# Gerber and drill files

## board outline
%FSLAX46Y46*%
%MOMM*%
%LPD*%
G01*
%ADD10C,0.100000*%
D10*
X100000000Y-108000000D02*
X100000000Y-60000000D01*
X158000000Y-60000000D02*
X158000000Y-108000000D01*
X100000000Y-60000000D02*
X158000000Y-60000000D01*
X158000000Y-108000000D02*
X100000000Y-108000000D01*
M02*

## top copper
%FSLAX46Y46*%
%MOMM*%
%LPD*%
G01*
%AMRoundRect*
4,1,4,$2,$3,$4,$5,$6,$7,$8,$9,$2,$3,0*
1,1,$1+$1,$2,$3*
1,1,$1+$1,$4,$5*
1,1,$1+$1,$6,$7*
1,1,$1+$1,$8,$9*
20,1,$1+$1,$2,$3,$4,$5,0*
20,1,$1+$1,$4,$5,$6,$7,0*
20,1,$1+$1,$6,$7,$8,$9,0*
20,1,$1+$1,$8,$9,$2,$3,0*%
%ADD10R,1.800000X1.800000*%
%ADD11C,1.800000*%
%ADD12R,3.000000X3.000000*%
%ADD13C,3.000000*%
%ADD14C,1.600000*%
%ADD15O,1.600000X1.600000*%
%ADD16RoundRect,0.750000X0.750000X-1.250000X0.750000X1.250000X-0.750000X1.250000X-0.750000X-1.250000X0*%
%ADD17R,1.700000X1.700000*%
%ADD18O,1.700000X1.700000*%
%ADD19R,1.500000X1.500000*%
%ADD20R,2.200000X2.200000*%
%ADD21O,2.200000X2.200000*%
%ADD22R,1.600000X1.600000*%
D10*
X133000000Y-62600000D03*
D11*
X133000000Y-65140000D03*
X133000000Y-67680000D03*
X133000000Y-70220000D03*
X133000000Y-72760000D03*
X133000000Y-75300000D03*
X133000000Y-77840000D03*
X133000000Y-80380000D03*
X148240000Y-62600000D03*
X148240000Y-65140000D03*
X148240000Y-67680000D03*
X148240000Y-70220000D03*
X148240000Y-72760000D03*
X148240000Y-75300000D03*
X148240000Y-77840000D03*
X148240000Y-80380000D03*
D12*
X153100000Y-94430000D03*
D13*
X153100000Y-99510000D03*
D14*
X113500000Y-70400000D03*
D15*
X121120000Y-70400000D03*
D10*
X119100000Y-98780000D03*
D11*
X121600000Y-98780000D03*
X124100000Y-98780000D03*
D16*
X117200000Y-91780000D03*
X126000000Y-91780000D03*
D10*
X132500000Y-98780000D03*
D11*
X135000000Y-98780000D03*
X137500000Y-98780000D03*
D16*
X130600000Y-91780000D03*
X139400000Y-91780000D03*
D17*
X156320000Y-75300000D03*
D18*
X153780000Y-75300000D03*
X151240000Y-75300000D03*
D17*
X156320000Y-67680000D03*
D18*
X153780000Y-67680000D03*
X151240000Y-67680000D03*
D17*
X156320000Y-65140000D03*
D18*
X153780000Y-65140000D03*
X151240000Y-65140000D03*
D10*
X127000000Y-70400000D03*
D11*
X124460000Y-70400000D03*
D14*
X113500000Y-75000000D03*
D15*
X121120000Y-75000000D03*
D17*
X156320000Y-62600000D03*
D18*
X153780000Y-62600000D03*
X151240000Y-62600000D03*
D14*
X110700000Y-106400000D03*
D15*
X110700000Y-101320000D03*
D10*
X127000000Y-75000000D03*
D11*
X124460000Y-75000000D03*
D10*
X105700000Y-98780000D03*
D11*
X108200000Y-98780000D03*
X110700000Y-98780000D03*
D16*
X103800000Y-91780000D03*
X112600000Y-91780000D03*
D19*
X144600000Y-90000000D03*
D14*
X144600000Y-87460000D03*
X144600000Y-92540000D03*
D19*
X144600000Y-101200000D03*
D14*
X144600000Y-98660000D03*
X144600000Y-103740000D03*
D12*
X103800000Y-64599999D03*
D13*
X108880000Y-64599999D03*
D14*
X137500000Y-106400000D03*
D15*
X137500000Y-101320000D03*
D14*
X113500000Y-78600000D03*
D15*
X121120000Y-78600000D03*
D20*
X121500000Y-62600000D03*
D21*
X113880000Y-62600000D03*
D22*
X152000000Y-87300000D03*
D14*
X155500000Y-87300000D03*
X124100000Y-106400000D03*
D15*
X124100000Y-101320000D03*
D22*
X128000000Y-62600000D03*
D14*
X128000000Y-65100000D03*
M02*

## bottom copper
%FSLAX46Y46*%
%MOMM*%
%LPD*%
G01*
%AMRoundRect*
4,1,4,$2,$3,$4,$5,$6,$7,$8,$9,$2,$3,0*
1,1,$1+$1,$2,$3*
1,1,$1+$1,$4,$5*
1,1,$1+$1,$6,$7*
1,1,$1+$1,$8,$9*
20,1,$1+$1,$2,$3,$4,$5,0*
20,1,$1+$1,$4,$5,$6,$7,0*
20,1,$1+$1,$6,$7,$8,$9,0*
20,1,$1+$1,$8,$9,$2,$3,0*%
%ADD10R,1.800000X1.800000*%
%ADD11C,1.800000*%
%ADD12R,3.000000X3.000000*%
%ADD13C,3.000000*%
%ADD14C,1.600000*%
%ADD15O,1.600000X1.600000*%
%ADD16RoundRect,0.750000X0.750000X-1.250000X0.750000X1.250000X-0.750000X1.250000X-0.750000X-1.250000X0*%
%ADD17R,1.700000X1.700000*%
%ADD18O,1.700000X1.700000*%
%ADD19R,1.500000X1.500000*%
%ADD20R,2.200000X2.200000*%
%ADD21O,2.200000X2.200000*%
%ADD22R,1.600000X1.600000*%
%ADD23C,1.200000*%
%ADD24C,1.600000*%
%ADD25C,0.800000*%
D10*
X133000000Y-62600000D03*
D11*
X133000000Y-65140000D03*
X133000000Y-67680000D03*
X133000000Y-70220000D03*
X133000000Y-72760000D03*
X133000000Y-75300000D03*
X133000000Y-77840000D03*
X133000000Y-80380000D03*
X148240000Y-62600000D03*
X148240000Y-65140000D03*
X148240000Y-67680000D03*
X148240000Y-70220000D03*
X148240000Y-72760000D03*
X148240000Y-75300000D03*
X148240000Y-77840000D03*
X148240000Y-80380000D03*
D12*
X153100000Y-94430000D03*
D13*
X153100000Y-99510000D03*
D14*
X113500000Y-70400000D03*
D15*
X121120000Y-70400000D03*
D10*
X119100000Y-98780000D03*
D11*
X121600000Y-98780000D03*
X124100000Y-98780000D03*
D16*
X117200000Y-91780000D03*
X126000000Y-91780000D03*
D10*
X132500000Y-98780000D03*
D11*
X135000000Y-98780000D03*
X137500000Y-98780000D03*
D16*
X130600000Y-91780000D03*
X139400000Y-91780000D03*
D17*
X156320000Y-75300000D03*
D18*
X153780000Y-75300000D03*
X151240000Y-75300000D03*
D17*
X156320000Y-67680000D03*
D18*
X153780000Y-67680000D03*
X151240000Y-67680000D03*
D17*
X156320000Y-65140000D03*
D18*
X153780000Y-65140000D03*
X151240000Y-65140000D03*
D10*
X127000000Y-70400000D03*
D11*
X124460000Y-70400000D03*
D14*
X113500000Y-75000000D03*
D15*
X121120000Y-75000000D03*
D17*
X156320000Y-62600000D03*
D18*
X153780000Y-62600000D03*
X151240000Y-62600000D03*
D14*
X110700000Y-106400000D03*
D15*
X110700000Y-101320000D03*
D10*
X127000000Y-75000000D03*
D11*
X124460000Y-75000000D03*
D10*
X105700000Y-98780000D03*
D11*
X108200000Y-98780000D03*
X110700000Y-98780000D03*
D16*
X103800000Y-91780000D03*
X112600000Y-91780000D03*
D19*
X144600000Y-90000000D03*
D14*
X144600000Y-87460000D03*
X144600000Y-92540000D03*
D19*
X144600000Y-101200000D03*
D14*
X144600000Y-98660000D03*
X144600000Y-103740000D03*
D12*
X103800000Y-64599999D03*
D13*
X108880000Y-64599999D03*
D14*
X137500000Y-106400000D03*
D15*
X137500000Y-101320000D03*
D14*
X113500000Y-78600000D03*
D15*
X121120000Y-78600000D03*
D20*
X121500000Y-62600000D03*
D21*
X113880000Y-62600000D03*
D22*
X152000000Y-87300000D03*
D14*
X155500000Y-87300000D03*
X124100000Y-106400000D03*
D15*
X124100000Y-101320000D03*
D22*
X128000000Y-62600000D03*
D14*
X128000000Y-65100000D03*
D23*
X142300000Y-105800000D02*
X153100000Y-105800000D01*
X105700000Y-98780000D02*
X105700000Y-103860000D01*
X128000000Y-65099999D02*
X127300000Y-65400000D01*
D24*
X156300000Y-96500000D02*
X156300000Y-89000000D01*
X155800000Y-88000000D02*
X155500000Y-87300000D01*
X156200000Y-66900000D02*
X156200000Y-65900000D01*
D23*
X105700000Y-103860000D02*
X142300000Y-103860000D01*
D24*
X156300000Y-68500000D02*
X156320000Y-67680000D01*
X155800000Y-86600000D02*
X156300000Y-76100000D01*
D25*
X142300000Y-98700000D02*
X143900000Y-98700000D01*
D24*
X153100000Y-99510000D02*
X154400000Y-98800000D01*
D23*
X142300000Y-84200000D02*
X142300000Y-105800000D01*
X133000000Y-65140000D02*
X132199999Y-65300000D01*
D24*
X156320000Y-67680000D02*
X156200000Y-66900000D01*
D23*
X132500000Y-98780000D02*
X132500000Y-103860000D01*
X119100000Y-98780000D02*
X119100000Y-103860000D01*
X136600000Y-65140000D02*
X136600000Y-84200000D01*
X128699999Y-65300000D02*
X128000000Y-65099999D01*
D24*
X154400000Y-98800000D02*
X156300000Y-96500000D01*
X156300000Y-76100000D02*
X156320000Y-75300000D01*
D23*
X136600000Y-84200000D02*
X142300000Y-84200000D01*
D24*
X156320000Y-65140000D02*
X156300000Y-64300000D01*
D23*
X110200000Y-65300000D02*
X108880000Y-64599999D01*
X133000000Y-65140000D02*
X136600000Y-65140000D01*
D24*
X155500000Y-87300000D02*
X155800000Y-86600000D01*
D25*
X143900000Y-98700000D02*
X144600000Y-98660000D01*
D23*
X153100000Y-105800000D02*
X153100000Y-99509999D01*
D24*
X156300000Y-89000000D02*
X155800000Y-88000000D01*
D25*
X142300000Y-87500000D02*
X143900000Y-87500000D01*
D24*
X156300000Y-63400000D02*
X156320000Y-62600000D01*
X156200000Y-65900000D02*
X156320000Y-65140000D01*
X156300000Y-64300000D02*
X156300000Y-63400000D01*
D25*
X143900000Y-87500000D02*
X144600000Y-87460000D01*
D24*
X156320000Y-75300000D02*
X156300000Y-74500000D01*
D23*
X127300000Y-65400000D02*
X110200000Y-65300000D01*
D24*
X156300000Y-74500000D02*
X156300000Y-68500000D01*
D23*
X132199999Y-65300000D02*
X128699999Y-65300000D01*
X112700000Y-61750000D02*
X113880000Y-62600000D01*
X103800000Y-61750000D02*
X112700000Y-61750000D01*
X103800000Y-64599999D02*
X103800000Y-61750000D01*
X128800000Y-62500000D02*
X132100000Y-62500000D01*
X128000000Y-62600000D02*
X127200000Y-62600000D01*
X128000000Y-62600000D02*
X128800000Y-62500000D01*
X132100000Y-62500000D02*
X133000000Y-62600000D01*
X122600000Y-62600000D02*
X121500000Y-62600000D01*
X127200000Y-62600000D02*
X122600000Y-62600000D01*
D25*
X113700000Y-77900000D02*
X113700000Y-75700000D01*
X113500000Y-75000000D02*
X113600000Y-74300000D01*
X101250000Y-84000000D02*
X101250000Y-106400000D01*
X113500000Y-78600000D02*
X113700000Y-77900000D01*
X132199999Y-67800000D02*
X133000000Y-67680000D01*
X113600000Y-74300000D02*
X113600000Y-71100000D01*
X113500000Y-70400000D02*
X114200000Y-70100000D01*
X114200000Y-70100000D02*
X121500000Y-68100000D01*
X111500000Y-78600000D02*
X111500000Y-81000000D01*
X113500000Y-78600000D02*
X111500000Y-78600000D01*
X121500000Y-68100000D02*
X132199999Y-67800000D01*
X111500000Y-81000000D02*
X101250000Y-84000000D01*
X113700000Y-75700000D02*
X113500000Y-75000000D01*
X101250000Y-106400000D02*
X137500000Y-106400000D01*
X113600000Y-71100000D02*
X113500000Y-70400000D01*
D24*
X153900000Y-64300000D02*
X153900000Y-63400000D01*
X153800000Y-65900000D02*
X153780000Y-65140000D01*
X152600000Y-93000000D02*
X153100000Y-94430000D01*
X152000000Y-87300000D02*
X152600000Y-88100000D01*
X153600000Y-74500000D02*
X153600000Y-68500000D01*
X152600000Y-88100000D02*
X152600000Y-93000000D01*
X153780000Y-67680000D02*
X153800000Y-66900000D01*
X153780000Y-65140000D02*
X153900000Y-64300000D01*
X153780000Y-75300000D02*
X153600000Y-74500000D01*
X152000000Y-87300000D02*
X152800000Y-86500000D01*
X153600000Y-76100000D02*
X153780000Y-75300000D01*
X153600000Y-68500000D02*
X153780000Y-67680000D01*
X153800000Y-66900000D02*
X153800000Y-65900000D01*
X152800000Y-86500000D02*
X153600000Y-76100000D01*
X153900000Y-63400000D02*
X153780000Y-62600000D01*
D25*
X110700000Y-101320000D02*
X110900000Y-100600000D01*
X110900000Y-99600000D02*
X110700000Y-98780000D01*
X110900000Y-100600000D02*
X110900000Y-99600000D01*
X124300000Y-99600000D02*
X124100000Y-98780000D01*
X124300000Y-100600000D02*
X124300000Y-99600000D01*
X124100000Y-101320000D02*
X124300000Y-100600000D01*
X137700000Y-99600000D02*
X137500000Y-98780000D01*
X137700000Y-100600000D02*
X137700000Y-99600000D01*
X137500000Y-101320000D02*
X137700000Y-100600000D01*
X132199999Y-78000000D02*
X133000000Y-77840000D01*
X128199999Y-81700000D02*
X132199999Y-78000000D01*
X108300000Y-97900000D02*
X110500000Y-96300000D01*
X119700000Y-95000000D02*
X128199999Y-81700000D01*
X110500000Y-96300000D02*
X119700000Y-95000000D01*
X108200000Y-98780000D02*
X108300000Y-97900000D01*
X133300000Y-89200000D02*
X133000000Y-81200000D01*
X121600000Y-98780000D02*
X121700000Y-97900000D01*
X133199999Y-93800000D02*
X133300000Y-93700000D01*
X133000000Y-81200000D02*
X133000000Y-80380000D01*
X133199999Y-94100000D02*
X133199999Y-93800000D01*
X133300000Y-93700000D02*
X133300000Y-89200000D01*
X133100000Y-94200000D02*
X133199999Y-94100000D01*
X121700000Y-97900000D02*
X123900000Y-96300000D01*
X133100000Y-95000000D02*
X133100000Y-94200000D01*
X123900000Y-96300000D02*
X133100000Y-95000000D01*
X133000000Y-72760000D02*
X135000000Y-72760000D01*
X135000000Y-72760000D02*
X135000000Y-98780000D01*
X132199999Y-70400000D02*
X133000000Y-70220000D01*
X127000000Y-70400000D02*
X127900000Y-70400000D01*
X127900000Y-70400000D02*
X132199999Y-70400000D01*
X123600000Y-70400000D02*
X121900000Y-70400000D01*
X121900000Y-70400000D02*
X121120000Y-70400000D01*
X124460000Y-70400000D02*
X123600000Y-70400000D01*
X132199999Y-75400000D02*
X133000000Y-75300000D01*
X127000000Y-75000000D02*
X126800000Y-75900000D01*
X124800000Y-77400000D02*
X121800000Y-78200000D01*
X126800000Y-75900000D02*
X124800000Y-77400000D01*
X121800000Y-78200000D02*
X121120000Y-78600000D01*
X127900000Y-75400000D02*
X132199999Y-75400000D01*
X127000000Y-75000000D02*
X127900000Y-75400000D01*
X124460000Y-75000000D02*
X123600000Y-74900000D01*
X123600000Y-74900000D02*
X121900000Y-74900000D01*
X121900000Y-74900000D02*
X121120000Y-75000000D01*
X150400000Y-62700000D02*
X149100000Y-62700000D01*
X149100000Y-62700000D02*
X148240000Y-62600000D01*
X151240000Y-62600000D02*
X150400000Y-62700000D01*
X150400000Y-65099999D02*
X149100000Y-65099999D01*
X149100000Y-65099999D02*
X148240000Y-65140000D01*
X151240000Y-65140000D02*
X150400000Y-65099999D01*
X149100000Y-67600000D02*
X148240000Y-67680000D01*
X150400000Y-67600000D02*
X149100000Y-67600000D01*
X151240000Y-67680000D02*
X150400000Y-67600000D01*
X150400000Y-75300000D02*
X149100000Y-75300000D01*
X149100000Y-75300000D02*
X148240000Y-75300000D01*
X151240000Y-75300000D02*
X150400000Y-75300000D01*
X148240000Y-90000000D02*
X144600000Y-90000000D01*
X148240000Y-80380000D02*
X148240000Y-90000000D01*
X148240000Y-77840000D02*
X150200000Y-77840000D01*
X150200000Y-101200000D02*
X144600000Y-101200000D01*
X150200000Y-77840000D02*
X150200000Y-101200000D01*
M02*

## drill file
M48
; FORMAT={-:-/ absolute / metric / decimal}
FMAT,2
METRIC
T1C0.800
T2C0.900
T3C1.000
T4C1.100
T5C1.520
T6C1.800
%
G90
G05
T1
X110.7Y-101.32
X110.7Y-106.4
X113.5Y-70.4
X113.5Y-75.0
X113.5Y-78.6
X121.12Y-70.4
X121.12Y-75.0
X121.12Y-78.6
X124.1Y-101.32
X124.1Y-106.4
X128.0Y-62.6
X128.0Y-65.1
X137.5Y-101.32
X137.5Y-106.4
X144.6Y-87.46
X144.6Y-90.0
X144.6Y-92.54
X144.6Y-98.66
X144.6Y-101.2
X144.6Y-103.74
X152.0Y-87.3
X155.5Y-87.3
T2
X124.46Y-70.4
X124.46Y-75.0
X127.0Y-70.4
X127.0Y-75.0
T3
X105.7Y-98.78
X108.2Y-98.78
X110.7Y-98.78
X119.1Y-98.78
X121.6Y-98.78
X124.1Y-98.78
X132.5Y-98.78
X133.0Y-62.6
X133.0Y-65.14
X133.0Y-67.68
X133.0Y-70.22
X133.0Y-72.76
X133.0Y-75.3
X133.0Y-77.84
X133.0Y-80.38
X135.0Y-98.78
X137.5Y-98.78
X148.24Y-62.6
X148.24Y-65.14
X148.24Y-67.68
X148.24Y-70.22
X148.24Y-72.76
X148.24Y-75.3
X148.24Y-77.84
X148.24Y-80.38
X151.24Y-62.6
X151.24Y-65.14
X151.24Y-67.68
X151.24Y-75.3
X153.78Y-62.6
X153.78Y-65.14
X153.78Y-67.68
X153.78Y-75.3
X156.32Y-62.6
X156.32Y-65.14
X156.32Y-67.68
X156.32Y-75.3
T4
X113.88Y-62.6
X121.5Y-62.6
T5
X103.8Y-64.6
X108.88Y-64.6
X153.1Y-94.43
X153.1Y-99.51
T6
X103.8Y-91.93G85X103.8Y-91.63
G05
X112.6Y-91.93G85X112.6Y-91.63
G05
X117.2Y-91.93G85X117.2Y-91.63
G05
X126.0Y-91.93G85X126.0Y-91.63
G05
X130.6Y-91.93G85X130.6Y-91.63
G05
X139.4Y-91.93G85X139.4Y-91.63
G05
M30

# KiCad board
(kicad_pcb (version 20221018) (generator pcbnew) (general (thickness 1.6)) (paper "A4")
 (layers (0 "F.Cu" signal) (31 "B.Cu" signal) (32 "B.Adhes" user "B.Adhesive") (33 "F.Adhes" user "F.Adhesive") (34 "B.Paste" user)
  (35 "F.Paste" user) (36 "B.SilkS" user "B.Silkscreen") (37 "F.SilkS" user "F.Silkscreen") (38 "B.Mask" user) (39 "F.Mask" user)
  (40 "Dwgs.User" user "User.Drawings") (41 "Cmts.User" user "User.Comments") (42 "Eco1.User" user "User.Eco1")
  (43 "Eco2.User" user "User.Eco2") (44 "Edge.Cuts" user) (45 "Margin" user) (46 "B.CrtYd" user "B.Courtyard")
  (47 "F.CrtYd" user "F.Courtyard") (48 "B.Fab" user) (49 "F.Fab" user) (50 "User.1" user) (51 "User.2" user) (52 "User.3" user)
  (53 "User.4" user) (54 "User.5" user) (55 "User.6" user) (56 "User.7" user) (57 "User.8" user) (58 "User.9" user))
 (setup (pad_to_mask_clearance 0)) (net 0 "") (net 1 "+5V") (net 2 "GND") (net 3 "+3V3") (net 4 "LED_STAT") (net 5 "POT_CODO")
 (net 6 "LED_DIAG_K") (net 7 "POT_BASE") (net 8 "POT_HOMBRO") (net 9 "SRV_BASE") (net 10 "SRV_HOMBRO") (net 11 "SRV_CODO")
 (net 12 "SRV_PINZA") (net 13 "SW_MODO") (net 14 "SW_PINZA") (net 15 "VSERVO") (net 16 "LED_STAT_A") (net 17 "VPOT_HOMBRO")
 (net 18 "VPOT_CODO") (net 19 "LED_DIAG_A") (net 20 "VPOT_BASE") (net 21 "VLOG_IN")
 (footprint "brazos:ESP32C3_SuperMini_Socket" (layer "F.Cu") (at 133 62.6)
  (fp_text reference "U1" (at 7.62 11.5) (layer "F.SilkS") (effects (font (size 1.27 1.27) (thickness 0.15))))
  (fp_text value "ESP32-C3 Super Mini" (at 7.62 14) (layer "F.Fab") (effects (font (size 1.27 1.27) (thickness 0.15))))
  (pad "1" thru_hole rect (at 0 0) (size 1.8 1.8) (drill 1) (layers "*.Cu" "*.Mask") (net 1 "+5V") (thermal_bridge_angle 45))
  (pad "2" thru_hole circle (at 0 2.54) (size 1.8 1.8) (drill 1) (layers "*.Cu" "*.Mask") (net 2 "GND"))
  (pad "3" thru_hole circle (at 0 5.08) (size 1.8 1.8) (drill 1) (layers "*.Cu" "*.Mask") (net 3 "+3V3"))
  (pad "4" thru_hole circle (at 0 7.62) (size 1.8 1.8) (drill 1) (layers "*.Cu" "*.Mask") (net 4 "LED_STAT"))
  (pad "5" thru_hole circle (at 0 10.16) (size 1.8 1.8) (drill 1) (layers "*.Cu" "*.Mask") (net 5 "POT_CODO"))
  (pad "6" thru_hole circle (at 0 12.7) (size 1.8 1.8) (drill 1) (layers "*.Cu" "*.Mask") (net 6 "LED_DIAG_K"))
  (pad "7" thru_hole circle (at 0 15.24) (size 1.8 1.8) (drill 1) (layers "*.Cu" "*.Mask") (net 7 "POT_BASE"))
  (pad "8" thru_hole circle (at 0 17.78) (size 1.8 1.8) (drill 1) (layers "*.Cu" "*.Mask") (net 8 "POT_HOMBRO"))
  (pad "9" thru_hole circle (at 15.24 0) (size 1.8 1.8) (drill 1) (layers "*.Cu" "*.Mask") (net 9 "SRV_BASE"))
  (pad "10" thru_hole circle (at 15.24 2.54) (size 1.8 1.8) (drill 1) (layers "*.Cu" "*.Mask") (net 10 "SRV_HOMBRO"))
  (pad "11" thru_hole circle (at 15.24 5.08) (size 1.8 1.8) (drill 1) (layers "*.Cu" "*.Mask") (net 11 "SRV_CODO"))
  (pad "12" thru_hole circle (at 15.24 7.62) (size 1.8 1.8) (drill 1) (layers "*.Cu" "*.Mask"))
  (pad "13" thru_hole circle (at 15.24 10.16) (size 1.8 1.8) (drill 1) (layers "*.Cu" "*.Mask"))
  (pad "14" thru_hole circle (at 15.24 12.7) (size 1.8 1.8) (drill 1) (layers "*.Cu" "*.Mask") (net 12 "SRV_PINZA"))
  (pad "15" thru_hole circle (at 15.24 15.24) (size 1.8 1.8) (drill 1) (layers "*.Cu" "*.Mask") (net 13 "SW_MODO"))
  (pad "16" thru_hole circle (at 15.24 17.78) (size 1.8 1.8) (drill 1) (layers "*.Cu" "*.Mask") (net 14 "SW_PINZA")))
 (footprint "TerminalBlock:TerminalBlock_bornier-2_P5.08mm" (layer "F.Cu") (at 153.1 94.43 -90)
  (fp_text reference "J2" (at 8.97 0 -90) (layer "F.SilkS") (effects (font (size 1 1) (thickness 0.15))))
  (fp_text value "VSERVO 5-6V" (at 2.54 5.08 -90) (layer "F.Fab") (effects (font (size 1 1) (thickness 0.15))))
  (pad "1" thru_hole rect (at 0 0 270) (size 3 3) (drill 1.52) (layers "*.Cu" "*.Mask") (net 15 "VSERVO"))
  (pad "2" thru_hole circle (at 5.08 0 270) (size 3 3) (drill 1.52) (layers "*.Cu" "*.Mask") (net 2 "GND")))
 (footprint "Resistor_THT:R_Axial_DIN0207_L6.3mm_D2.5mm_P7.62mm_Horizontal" (layer "F.Cu") (at 113.5 70.4)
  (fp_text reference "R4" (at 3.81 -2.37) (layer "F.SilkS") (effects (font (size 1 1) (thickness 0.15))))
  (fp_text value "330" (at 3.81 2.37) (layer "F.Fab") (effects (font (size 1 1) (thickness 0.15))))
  (pad "1" thru_hole circle (at 0 0) (size 1.6 1.6) (drill 0.8) (layers "*.Cu" "*.Mask") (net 3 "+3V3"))
  (pad "2" thru_hole oval (at 7.62 0) (size 1.6 1.6) (drill 0.8) (layers "*.Cu" "*.Mask") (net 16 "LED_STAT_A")))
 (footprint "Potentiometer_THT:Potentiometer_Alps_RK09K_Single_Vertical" (layer "F.Cu") (at 119.1 98.78 90)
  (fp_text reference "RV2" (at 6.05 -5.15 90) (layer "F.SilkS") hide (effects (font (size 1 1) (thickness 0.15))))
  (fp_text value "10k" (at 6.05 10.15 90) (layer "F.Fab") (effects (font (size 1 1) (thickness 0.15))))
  (pad "1" thru_hole rect (at 0 0 90) (size 1.8 1.8) (drill 1) (layers "*.Cu" "*.Mask") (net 2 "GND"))
  (pad "2" thru_hole circle (at 0 2.5 90) (size 1.8 1.8) (drill 1) (layers "*.Cu" "*.Mask") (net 8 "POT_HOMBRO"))
  (pad "3" thru_hole circle (at 0 5 90) (size 1.8 1.8) (drill 1) (layers "*.Cu" "*.Mask") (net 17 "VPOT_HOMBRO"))
  (pad "MP" thru_hole roundrect (at 7 -1.9 90) (size 4 3) (drill oval 2.1 1.8) (layers "*.Cu" "*.Mask") (roundrect_rratio 0.25))
  (pad "MP" thru_hole roundrect (at 7 6.9 90) (size 4 3) (drill oval 2.1 1.8) (layers "*.Cu" "*.Mask") (roundrect_rratio 0.25)))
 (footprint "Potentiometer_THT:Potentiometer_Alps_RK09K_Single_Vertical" (layer "F.Cu") (at 132.5 98.78 90)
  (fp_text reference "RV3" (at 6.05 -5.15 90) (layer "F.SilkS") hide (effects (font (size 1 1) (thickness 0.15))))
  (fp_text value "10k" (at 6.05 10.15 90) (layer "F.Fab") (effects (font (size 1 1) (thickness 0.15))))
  (pad "1" thru_hole rect (at 0 0 90) (size 1.8 1.8) (drill 1) (layers "*.Cu" "*.Mask") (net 2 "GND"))
  (pad "2" thru_hole circle (at 0 2.5 90) (size 1.8 1.8) (drill 1) (layers "*.Cu" "*.Mask") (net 5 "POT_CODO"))
  (pad "3" thru_hole circle (at 0 5 90) (size 1.8 1.8) (drill 1) (layers "*.Cu" "*.Mask") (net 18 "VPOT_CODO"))
  (pad "MP" thru_hole roundrect (at 7 -1.9 90) (size 4 3) (drill oval 2.1 1.8) (layers "*.Cu" "*.Mask") (roundrect_rratio 0.25))
  (pad "MP" thru_hole roundrect (at 7 6.9 90) (size 4 3) (drill oval 2.1 1.8) (layers "*.Cu" "*.Mask") (roundrect_rratio 0.25)))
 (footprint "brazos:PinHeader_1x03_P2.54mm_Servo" (layer "F.Cu") (at 156.32 75.3 -90)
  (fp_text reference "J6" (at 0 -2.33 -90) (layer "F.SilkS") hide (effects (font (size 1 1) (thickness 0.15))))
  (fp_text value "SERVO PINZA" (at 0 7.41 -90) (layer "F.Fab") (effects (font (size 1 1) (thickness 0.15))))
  (pad "1" thru_hole rect (at 0 0 270) (size 1.7 1.7) (drill 1) (layers "*.Cu" "*.Mask") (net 2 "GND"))
  (pad "2" thru_hole oval (at 0 2.54 270) (size 1.7 1.7) (drill 1) (layers "*.Cu" "*.Mask") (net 15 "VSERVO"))
  (pad "3" thru_hole oval (at 0 5.08 270) (size 1.7 1.7) (drill 1) (layers "*.Cu" "*.Mask") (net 12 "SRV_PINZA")))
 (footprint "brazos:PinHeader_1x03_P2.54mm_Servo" (layer "F.Cu") (at 156.32 67.68 -90)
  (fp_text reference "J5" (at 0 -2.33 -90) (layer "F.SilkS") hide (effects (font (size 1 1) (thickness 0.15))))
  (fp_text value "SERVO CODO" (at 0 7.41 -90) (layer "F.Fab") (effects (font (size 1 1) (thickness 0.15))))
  (pad "1" thru_hole rect (at 0 0 270) (size 1.7 1.7) (drill 1) (layers "*.Cu" "*.Mask") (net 2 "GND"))
  (pad "2" thru_hole oval (at 0 2.54 270) (size 1.7 1.7) (drill 1) (layers "*.Cu" "*.Mask") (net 15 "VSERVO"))
  (pad "3" thru_hole oval (at 0 5.08 270) (size 1.7 1.7) (drill 1) (layers "*.Cu" "*.Mask") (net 11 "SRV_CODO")))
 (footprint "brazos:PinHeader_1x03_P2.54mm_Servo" (layer "F.Cu") (at 156.32 65.14 -90)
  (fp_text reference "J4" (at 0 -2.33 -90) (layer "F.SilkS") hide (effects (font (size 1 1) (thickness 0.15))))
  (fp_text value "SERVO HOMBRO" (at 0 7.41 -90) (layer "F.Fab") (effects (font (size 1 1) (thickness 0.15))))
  (pad "1" thru_hole rect (at 0 0 270) (size 1.7 1.7) (drill 1) (layers "*.Cu" "*.Mask") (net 2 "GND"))
  (pad "2" thru_hole oval (at 0 2.54 270) (size 1.7 1.7) (drill 1) (layers "*.Cu" "*.Mask") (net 15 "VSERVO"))
  (pad "3" thru_hole oval (at 0 5.08 270) (size 1.7 1.7) (drill 1) (layers "*.Cu" "*.Mask") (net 10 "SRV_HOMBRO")))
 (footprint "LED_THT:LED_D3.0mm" (layer "F.Cu") (at 127 70.4 180)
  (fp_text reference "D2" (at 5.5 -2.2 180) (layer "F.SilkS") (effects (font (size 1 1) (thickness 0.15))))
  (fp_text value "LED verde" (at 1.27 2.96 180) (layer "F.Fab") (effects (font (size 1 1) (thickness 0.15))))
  (pad "1" thru_hole rect (at 0 0 180) (size 1.8 1.8) (drill 0.9) (layers "*.Cu" "*.Mask") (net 4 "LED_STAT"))
  (pad "2" thru_hole circle (at 2.54 0 180) (size 1.8 1.8) (drill 0.9) (layers "*.Cu" "*.Mask") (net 16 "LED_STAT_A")))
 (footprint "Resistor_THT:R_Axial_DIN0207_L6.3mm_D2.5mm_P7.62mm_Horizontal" (layer "F.Cu") (at 113.5 75)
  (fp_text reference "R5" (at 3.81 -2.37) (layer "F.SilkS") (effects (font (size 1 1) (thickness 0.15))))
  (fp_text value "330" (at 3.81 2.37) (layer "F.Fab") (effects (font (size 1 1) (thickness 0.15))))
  (pad "1" thru_hole circle (at 0 0) (size 1.6 1.6) (drill 0.8) (layers "*.Cu" "*.Mask") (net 3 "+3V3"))
  (pad "2" thru_hole oval (at 7.62 0) (size 1.6 1.6) (drill 0.8) (layers "*.Cu" "*.Mask") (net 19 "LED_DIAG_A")))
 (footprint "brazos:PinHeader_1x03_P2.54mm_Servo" (layer "F.Cu") (at 156.32 62.6 -90)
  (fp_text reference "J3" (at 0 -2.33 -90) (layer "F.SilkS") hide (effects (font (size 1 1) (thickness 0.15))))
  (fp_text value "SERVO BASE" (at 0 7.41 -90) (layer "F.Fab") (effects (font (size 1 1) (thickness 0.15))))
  (pad "1" thru_hole rect (at 0 0 270) (size 1.7 1.7) (drill 1) (layers "*.Cu" "*.Mask") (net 2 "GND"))
  (pad "2" thru_hole oval (at 0 2.54 270) (size 1.7 1.7) (drill 1) (layers "*.Cu" "*.Mask") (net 15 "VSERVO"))
  (pad "3" thru_hole oval (at 0 5.08 270) (size 1.7 1.7) (drill 1) (layers "*.Cu" "*.Mask") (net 9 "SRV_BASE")))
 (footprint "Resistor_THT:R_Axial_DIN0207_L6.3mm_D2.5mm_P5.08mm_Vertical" (layer "F.Cu") (at 110.7 106.4 90)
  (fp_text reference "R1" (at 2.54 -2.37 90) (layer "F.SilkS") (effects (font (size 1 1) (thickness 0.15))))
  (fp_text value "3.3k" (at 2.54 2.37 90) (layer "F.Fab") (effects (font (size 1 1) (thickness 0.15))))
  (pad "1" thru_hole circle (at 0 0 90) (size 1.6 1.6) (drill 0.8) (layers "*.Cu" "*.Mask") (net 3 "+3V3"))
  (pad "2" thru_hole oval (at 5.08 0 90) (size 1.6 1.6) (drill 0.8) (layers "*.Cu" "*.Mask") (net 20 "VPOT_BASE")))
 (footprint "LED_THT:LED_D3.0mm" (layer "F.Cu") (at 127 75 180)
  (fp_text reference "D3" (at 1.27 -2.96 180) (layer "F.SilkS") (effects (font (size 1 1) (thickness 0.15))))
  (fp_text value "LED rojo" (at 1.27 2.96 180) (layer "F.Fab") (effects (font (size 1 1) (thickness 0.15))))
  (pad "1" thru_hole rect (at 0 0 180) (size 1.8 1.8) (drill 0.9) (layers "*.Cu" "*.Mask") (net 6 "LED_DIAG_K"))
  (pad "2" thru_hole circle (at 2.54 0 180) (size 1.8 1.8) (drill 0.9) (layers "*.Cu" "*.Mask") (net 19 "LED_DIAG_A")))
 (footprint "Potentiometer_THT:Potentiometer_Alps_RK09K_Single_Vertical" (layer "F.Cu") (at 105.7 98.78 90)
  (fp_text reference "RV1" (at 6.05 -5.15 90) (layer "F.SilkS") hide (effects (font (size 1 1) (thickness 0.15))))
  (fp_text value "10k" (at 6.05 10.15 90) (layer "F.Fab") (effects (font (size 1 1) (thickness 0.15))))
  (pad "1" thru_hole rect (at 0 0 90) (size 1.8 1.8) (drill 1) (layers "*.Cu" "*.Mask") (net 2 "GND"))
  (pad "2" thru_hole circle (at 0 2.5 90) (size 1.8 1.8) (drill 1) (layers "*.Cu" "*.Mask") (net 7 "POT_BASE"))
  (pad "3" thru_hole circle (at 0 5 90) (size 1.8 1.8) (drill 1) (layers "*.Cu" "*.Mask") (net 20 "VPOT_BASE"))
  (pad "MP" thru_hole roundrect (at 7 -1.9 90) (size 4 3) (drill oval 2.1 1.8) (layers "*.Cu" "*.Mask") (roundrect_rratio 0.25))
  (pad "MP" thru_hole roundrect (at 7 6.9 90) (size 4 3) (drill oval 2.1 1.8) (layers "*.Cu" "*.Mask") (roundrect_rratio 0.25)))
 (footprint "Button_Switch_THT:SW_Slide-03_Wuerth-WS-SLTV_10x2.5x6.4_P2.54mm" (layer "F.Cu") (at 144.6 90 -90)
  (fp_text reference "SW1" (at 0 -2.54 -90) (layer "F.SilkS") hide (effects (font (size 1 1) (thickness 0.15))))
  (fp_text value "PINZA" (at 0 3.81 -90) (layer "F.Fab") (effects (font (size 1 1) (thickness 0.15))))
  (pad "1" thru_hole rect (at 0 0 270) (size 1.5 1.5) (drill 0.8) (layers "*.Cu" "*.Mask") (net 14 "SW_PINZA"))
  (pad "2" thru_hole circle (at -2.54 0 270) (size 1.6 1.6) (drill 0.8) (layers "*.Cu" "*.Mask") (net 2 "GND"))
  (pad "3" thru_hole circle (at 2.54 0 270) (size 1.6 1.6) (drill 0.8) (layers "*.Cu" "*.Mask")))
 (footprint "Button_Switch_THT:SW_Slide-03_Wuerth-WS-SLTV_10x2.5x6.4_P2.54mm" (layer "F.Cu") (at 144.6 101.2 -90)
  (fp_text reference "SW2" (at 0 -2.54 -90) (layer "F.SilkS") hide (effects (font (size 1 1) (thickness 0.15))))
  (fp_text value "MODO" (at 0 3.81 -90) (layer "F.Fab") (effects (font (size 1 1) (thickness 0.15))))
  (pad "1" thru_hole rect (at 0 0 270) (size 1.5 1.5) (drill 0.8) (layers "*.Cu" "*.Mask") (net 13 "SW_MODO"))
  (pad "2" thru_hole circle (at -2.54 0 270) (size 1.6 1.6) (drill 0.8) (layers "*.Cu" "*.Mask") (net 2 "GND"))
  (pad "3" thru_hole circle (at 2.54 0 270) (size 1.6 1.6) (drill 0.8) (layers "*.Cu" "*.Mask")))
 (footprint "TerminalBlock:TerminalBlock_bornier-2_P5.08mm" (layer "F.Cu") (at 103.8 64.599999)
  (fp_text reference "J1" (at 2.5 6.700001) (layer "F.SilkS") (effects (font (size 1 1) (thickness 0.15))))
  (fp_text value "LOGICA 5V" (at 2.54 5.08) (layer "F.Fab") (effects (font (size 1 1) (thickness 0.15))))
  (pad "1" thru_hole rect (at 0 0) (size 3 3) (drill 1.52) (layers "*.Cu" "*.Mask") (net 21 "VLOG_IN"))
  (pad "2" thru_hole circle (at 5.08 0) (size 3 3) (drill 1.52) (layers "*.Cu" "*.Mask") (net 2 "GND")))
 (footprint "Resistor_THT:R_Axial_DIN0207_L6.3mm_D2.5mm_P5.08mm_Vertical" (layer "F.Cu") (at 137.5 106.4 90)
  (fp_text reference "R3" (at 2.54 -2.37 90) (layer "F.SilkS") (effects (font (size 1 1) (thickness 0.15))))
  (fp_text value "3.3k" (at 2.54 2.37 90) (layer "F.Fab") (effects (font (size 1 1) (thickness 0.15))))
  (pad "1" thru_hole circle (at 0 0 90) (size 1.6 1.6) (drill 0.8) (layers "*.Cu" "*.Mask") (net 3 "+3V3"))
  (pad "2" thru_hole oval (at 5.08 0 90) (size 1.6 1.6) (drill 0.8) (layers "*.Cu" "*.Mask") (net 18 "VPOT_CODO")))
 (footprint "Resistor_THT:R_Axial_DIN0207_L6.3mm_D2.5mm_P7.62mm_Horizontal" (layer "F.Cu") (at 113.5 78.6)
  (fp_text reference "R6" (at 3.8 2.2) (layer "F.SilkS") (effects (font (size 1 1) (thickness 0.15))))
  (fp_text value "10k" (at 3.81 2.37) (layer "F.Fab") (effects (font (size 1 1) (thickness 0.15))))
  (pad "1" thru_hole circle (at 0 0) (size 1.6 1.6) (drill 0.8) (layers "*.Cu" "*.Mask") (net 3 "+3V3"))
  (pad "2" thru_hole oval (at 7.62 0) (size 1.6 1.6) (drill 0.8) (layers "*.Cu" "*.Mask") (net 6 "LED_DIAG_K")))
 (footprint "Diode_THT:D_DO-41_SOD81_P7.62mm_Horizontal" (layer "F.Cu") (at 121.5 62.6 180)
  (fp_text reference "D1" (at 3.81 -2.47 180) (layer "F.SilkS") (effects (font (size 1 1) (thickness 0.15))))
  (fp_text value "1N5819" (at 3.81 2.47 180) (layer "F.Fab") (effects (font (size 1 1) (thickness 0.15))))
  (pad "1" thru_hole rect (at 0 0 180) (size 2.2 2.2) (drill 1.1) (layers "*.Cu" "*.Mask") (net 1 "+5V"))
  (pad "2" thru_hole oval (at 7.62 0 180) (size 2.2 2.2) (drill 1.1) (layers "*.Cu" "*.Mask") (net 21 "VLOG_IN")))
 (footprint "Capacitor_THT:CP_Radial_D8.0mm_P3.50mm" (layer "F.Cu") (at 152 87.3)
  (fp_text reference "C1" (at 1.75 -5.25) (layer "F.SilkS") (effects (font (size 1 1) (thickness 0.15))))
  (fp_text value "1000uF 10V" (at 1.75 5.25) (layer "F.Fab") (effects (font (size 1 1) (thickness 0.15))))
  (pad "1" thru_hole rect (at 0 0) (size 1.6 1.6) (drill 0.8) (layers "*.Cu" "*.Mask") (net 15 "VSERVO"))
  (pad "2" thru_hole circle (at 3.5 0) (size 1.6 1.6) (drill 0.8) (layers "*.Cu" "*.Mask") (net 2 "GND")))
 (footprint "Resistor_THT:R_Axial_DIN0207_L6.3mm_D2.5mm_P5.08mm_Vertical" (layer "F.Cu") (at 124.1 106.4 90)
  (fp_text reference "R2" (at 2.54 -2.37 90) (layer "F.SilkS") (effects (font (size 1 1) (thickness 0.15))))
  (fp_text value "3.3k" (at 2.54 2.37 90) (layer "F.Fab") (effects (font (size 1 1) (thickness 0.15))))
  (pad "1" thru_hole circle (at 0 0 90) (size 1.6 1.6) (drill 0.8) (layers "*.Cu" "*.Mask") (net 3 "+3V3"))
  (pad "2" thru_hole oval (at 5.08 0 90) (size 1.6 1.6) (drill 0.8) (layers "*.Cu" "*.Mask") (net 17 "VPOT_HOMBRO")))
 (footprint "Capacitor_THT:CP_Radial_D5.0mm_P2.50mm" (layer "F.Cu") (at 128 62.6 -90)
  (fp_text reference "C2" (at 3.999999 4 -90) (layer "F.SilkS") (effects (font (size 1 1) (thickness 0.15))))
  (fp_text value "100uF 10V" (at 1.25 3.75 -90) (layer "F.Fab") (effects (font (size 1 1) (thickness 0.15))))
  (pad "1" thru_hole rect (at 0 0 270) (size 1.6 1.6) (drill 0.8) (layers "*.Cu" "*.Mask") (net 1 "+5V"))
  (pad "2" thru_hole circle (at 2.5 0 270) (size 1.6 1.6) (drill 0.8) (layers "*.Cu" "*.Mask") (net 2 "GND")))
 (gr_line (start 100 108) (end 100 60) (stroke (width 0.1) (type default)) (layer "Edge.Cuts"))
 (gr_line (start 158 60) (end 158 108) (stroke (width 0.1) (type default)) (layer "Edge.Cuts"))
 (gr_line (start 100 60) (end 158 60) (stroke (width 0.1) (type default)) (layer "Edge.Cuts"))
 (gr_line (start 158 108) (end 100 108) (stroke (width 0.1) (type default)) (layer "Edge.Cuts"))
 (segment (start 142.3 105.8) (end 153.1 105.8) (width 1.2) (layer "B.Cu") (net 2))
 (segment (start 105.7 98.78) (end 105.7 103.86) (width 1.2) (layer "B.Cu") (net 2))
 (segment (start 128 65.099999) (end 127.3 65.4) (width 1.2) (layer "B.Cu") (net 2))
 (segment (start 156.3 96.5) (end 156.3 89) (width 1.6) (layer "B.Cu") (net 2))
 (segment (start 155.8 88) (end 155.5 87.3) (width 1.6) (layer "B.Cu") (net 2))
 (segment (start 156.2 66.9) (end 156.2 65.9) (width 1.6) (layer "B.Cu") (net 2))
 (segment (start 105.7 103.86) (end 142.3 103.86) (width 1.2) (layer "B.Cu") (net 2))
 (segment (start 156.3 68.5) (end 156.32 67.68) (width 1.6) (layer "B.Cu") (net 2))
 (segment (start 155.8 86.6) (end 156.3 76.1) (width 1.6) (layer "B.Cu") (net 2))
 (segment (start 142.3 98.7) (end 143.9 98.7) (width 0.8) (layer "B.Cu") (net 2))
 (segment (start 153.1 99.51) (end 154.4 98.8) (width 1.6) (layer "B.Cu") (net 2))
 (segment (start 142.3 84.2) (end 142.3 105.8) (width 1.2) (layer "B.Cu") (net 2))
 (segment (start 133 65.14) (end 132.199999 65.3) (width 1.2) (layer "B.Cu") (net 2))
 (segment (start 156.32 67.68) (end 156.2 66.9) (width 1.6) (layer "B.Cu") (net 2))
 (segment (start 132.5 98.78) (end 132.5 103.86) (width 1.2) (layer "B.Cu") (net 2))
 (segment (start 119.1 98.78) (end 119.1 103.86) (width 1.2) (layer "B.Cu") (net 2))
 (segment (start 136.6 65.14) (end 136.6 84.2) (width 1.2) (layer "B.Cu") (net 2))
 (segment (start 128.699999 65.3) (end 128 65.099999) (width 1.2) (layer "B.Cu") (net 2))
 (segment (start 154.4 98.8) (end 156.3 96.5) (width 1.6) (layer "B.Cu") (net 2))
 (segment (start 156.3 76.1) (end 156.32 75.3) (width 1.6) (layer "B.Cu") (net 2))
 (segment (start 136.6 84.2) (end 142.3 84.2) (width 1.2) (layer "B.Cu") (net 2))
 (segment (start 156.32 65.14) (end 156.3 64.3) (width 1.6) (layer "B.Cu") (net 2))
 (segment (start 110.2 65.3) (end 108.88 64.599999) (width 1.2) (layer "B.Cu") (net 2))
 (segment (start 133 65.14) (end 136.6 65.14) (width 1.2) (layer "B.Cu") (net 2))
 (segment (start 155.5 87.3) (end 155.8 86.6) (width 1.6) (layer "B.Cu") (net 2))
 (segment (start 143.9 98.7) (end 144.6 98.66) (width 0.8) (layer "B.Cu") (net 2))
 (segment (start 153.1 105.8) (end 153.1 99.509999) (width 1.2) (layer "B.Cu") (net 2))
 (segment (start 156.3 89) (end 155.8 88) (width 1.6) (layer "B.Cu") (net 2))
 (segment (start 142.3 87.5) (end 143.9 87.5) (width 0.8) (layer "B.Cu") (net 2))
 (segment (start 156.3 63.4) (end 156.32 62.6) (width 1.6) (layer "B.Cu") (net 2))
 (segment (start 156.2 65.9) (end 156.32 65.14) (width 1.6) (layer "B.Cu") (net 2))
 (segment (start 156.3 64.3) (end 156.3 63.4) (width 1.6) (layer "B.Cu") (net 2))
 (segment (start 143.9 87.5) (end 144.6 87.46) (width 0.8) (layer "B.Cu") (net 2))
 (segment (start 156.32 75.3) (end 156.3 74.5) (width 1.6) (layer "B.Cu") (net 2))
 (segment (start 127.3 65.4) (end 110.2 65.3) (width 1.2) (layer "B.Cu") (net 2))
 (segment (start 156.3 74.5) (end 156.3 68.5) (width 1.6) (layer "B.Cu") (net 2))
 (segment (start 132.199999 65.3) (end 128.699999 65.3) (width 1.2) (layer "B.Cu") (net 2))
 (segment (start 112.7 61.75) (end 113.88 62.6) (width 1.2) (layer "B.Cu") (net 21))
 (segment (start 103.8 61.75) (end 112.7 61.75) (width 1.2) (layer "B.Cu") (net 21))
 (segment (start 103.8 64.599999) (end 103.8 61.75) (width 1.2) (layer "B.Cu") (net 21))
 (segment (start 128.8 62.5) (end 132.1 62.5) (width 1.2) (layer "B.Cu") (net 1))
 (segment (start 128 62.6) (end 127.2 62.6) (width 1.2) (layer "B.Cu") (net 1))
 (segment (start 128 62.6) (end 128.8 62.5) (width 1.2) (layer "B.Cu") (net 1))
 (segment (start 132.1 62.5) (end 133 62.6) (width 1.2) (layer "B.Cu") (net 1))
 (segment (start 122.6 62.6) (end 121.5 62.6) (width 1.2) (layer "B.Cu") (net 1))
 (segment (start 127.2 62.6) (end 122.6 62.6) (width 1.2) (layer "B.Cu") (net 1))
 (segment (start 113.7 77.9) (end 113.7 75.7) (width 0.8) (layer "B.Cu") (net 3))
 (segment (start 113.5 75) (end 113.6 74.3) (width 0.8) (layer "B.Cu") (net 3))
 (segment (start 101.25 84) (end 101.25 106.4) (width 0.8) (layer "B.Cu") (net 3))
 (segment (start 113.5 78.6) (end 113.7 77.9) (width 0.8) (layer "B.Cu") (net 3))
 (segment (start 132.199999 67.8) (end 133 67.68) (width 0.8) (layer "B.Cu") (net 3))
 (segment (start 113.6 74.3) (end 113.6 71.1) (width 0.8) (layer "B.Cu") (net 3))
 (segment (start 113.5 70.4) (end 114.2 70.1) (width 0.8) (layer "B.Cu") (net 3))
 (segment (start 114.2 70.1) (end 121.5 68.1) (width 0.8) (layer "B.Cu") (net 3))
 (segment (start 111.5 78.6) (end 111.5 81) (width 0.8) (layer "B.Cu") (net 3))
 (segment (start 113.5 78.6) (end 111.5 78.6) (width 0.8) (layer "B.Cu") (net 3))
 (segment (start 121.5 68.1) (end 132.199999 67.8) (width 0.8) (layer "B.Cu") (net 3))
 (segment (start 111.5 81) (end 101.25 84) (width 0.8) (layer "B.Cu") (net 3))
 (segment (start 113.7 75.7) (end 113.5 75) (width 0.8) (layer "B.Cu") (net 3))
 (segment (start 101.25 106.4) (end 137.5 106.4) (width 0.8) (layer "B.Cu") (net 3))
 (segment (start 113.6 71.1) (end 113.5 70.4) (width 0.8) (layer "B.Cu") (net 3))
 (segment (start 153.9 64.3) (end 153.9 63.4) (width 1.6) (layer "B.Cu") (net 15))
 (segment (start 153.8 65.9) (end 153.78 65.14) (width 1.6) (layer "B.Cu") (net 15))
 (segment (start 152.6 93) (end 153.1 94.43) (width 1.6) (layer "B.Cu") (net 15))
 (segment (start 152 87.3) (end 152.6 88.1) (width 1.6) (layer "B.Cu") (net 15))
 (segment (start 153.6 74.5) (end 153.6 68.5) (width 1.6) (layer "B.Cu") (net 15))
 (segment (start 152.6 88.1) (end 152.6 93) (width 1.6) (layer "B.Cu") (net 15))
 (segment (start 153.78 67.68) (end 153.8 66.9) (width 1.6) (layer "B.Cu") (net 15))
 (segment (start 153.78 65.14) (end 153.9 64.3) (width 1.6) (layer "B.Cu") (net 15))
 (segment (start 153.78 75.3) (end 153.6 74.5) (width 1.6) (layer "B.Cu") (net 15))
 (segment (start 152 87.3) (end 152.8 86.5) (width 1.6) (layer "B.Cu") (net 15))
 (segment (start 153.6 76.1) (end 153.78 75.3) (width 1.6) (layer "B.Cu") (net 15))
 (segment (start 153.6 68.5) (end 153.78 67.68) (width 1.6) (layer "B.Cu") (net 15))
 (segment (start 153.8 66.9) (end 153.8 65.9) (width 1.6) (layer "B.Cu") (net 15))
 (segment (start 152.8 86.5) (end 153.6 76.1) (width 1.6) (layer "B.Cu") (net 15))
 (segment (start 153.9 63.4) (end 153.78 62.6) (width 1.6) (layer "B.Cu") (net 15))
 (segment (start 110.7 101.32) (end 110.9 100.6) (width 0.8) (layer "B.Cu") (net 20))
 (segment (start 110.9 99.6) (end 110.7 98.78) (width 0.8) (layer "B.Cu") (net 20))
 (segment (start 110.9 100.6) (end 110.9 99.6) (width 0.8) (layer "B.Cu") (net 20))
 (segment (start 124.3 99.6) (end 124.1 98.78) (width 0.8) (layer "B.Cu") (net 17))
 (segment (start 124.3 100.6) (end 124.3 99.6) (width 0.8) (layer "B.Cu") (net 17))
 (segment (start 124.1 101.32) (end 124.3 100.6) (width 0.8) (layer "B.Cu") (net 17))
 (segment (start 137.7 99.6) (end 137.5 98.78) (width 0.8) (layer "B.Cu") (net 18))
 (segment (start 137.7 100.6) (end 137.7 99.6) (width 0.8) (layer "B.Cu") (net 18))
 (segment (start 137.5 101.32) (end 137.7 100.6) (width 0.8) (layer "B.Cu") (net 18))
 (segment (start 132.199999 78) (end 133 77.84) (width 0.8) (layer "B.Cu") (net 7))
 (segment (start 128.199999 81.7) (end 132.199999 78) (width 0.8) (layer "B.Cu") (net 7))
 (segment (start 108.3 97.9) (end 110.5 96.3) (width 0.8) (layer "B.Cu") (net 7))
 (segment (start 119.7 95) (end 128.199999 81.7) (width 0.8) (layer "B.Cu") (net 7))
 (segment (start 110.5 96.3) (end 119.7 95) (width 0.8) (layer "B.Cu") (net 7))
 (segment (start 108.2 98.78) (end 108.3 97.9) (width 0.8) (layer "B.Cu") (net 7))
 (segment (start 133.3 89.2) (end 133 81.2) (width 0.8) (layer "B.Cu") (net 8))
 (segment (start 121.6 98.78) (end 121.7 97.9) (width 0.8) (layer "B.Cu") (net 8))
 (segment (start 133.199999 93.8) (end 133.3 93.7) (width 0.8) (layer "B.Cu") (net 8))
 (segment (start 133 81.2) (end 133 80.38) (width 0.8) (layer "B.Cu") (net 8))
 (segment (start 133.199999 94.1) (end 133.199999 93.8) (width 0.8) (layer "B.Cu") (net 8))
 (segment (start 133.3 93.7) (end 133.3 89.2) (width 0.8) (layer "B.Cu") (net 8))
 (segment (start 133.1 94.2) (end 133.199999 94.1) (width 0.8) (layer "B.Cu") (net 8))
 (segment (start 121.7 97.9) (end 123.9 96.3) (width 0.8) (layer "B.Cu") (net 8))
 (segment (start 133.1 95) (end 133.1 94.2) (width 0.8) (layer "B.Cu") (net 8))
 (segment (start 123.9 96.3) (end 133.1 95) (width 0.8) (layer "B.Cu") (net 8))
 (segment (start 133 72.76) (end 135 72.76) (width 0.8) (layer "B.Cu") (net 5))
 (segment (start 135 72.76) (end 135 98.78) (width 0.8) (layer "B.Cu") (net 5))
 (segment (start 132.199999 70.4) (end 133 70.22) (width 0.8) (layer "B.Cu") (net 4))
 (segment (start 127 70.4) (end 127.9 70.4) (width 0.8) (layer "B.Cu") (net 4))
 (segment (start 127.9 70.4) (end 132.199999 70.4) (width 0.8) (layer "B.Cu") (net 4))
 (segment (start 123.6 70.4) (end 121.9 70.4) (width 0.8) (layer "B.Cu") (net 16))
 (segment (start 121.9 70.4) (end 121.12 70.4) (width 0.8) (layer "B.Cu") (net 16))
 (segment (start 124.46 70.4) (end 123.6 70.4) (width 0.8) (layer "B.Cu") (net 16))
 (segment (start 132.199999 75.4) (end 133 75.3) (width 0.8) (layer "B.Cu") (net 6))
 (segment (start 127 75) (end 126.8 75.9) (width 0.8) (layer "B.Cu") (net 6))
 (segment (start 124.8 77.4) (end 121.8 78.2) (width 0.8) (layer "B.Cu") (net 6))
 (segment (start 126.8 75.9) (end 124.8 77.4) (width 0.8) (layer "B.Cu") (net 6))
 (segment (start 121.8 78.2) (end 121.12 78.6) (width 0.8) (layer "B.Cu") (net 6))
 (segment (start 127.9 75.4) (end 132.199999 75.4) (width 0.8) (layer "B.Cu") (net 6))
 (segment (start 127 75) (end 127.9 75.4) (width 0.8) (layer "B.Cu") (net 6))
 (segment (start 124.46 75) (end 123.6 74.9) (width 0.8) (layer "B.Cu") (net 19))
 (segment (start 123.6 74.9) (end 121.9 74.9) (width 0.8) (layer "B.Cu") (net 19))
 (segment (start 121.9 74.9) (end 121.12 75) (width 0.8) (layer "B.Cu") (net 19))
 (segment (start 150.4 62.7) (end 149.1 62.7) (width 0.8) (layer "B.Cu") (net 9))
 (segment (start 149.1 62.7) (end 148.24 62.6) (width 0.8) (layer "B.Cu") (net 9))
 (segment (start 151.24 62.6) (end 150.4 62.7) (width 0.8) (layer "B.Cu") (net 9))
 (segment (start 150.4 65.099999) (end 149.1 65.099999) (width 0.8) (layer "B.Cu") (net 10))
 (segment (start 149.1 65.099999) (end 148.24 65.14) (width 0.8) (layer "B.Cu") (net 10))
 (segment (start 151.24 65.14) (end 150.4 65.099999) (width 0.8) (layer "B.Cu") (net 10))
 (segment (start 149.1 67.6) (end 148.24 67.68) (width 0.8) (layer "B.Cu") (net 11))
 (segment (start 150.4 67.6) (end 149.1 67.6) (width 0.8) (layer "B.Cu") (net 11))
 (segment (start 151.24 67.68) (end 150.4 67.6) (width 0.8) (layer "B.Cu") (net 11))
 (segment (start 150.4 75.3) (end 149.1 75.3) (width 0.8) (layer "B.Cu") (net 12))
 (segment (start 149.1 75.3) (end 148.24 75.3) (width 0.8) (layer "B.Cu") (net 12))
 (segment (start 151.24 75.3) (end 150.4 75.3) (width 0.8) (layer "B.Cu") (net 12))
 (segment (start 148.24 90) (end 144.6 90) (width 0.8) (layer "B.Cu") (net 14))
 (segment (start 148.24 80.38) (end 148.24 90) (width 0.8) (layer "B.Cu") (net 14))
 (segment (start 148.24 77.84) (end 150.2 77.84) (width 0.8) (layer "B.Cu") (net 13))
 (segment (start 150.2 101.2) (end 144.6 101.2) (width 0.8) (layer "B.Cu") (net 13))
 (segment (start 150.2 77.84) (end 150.2 101.2) (width 0.8) (layer "B.Cu") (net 13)))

